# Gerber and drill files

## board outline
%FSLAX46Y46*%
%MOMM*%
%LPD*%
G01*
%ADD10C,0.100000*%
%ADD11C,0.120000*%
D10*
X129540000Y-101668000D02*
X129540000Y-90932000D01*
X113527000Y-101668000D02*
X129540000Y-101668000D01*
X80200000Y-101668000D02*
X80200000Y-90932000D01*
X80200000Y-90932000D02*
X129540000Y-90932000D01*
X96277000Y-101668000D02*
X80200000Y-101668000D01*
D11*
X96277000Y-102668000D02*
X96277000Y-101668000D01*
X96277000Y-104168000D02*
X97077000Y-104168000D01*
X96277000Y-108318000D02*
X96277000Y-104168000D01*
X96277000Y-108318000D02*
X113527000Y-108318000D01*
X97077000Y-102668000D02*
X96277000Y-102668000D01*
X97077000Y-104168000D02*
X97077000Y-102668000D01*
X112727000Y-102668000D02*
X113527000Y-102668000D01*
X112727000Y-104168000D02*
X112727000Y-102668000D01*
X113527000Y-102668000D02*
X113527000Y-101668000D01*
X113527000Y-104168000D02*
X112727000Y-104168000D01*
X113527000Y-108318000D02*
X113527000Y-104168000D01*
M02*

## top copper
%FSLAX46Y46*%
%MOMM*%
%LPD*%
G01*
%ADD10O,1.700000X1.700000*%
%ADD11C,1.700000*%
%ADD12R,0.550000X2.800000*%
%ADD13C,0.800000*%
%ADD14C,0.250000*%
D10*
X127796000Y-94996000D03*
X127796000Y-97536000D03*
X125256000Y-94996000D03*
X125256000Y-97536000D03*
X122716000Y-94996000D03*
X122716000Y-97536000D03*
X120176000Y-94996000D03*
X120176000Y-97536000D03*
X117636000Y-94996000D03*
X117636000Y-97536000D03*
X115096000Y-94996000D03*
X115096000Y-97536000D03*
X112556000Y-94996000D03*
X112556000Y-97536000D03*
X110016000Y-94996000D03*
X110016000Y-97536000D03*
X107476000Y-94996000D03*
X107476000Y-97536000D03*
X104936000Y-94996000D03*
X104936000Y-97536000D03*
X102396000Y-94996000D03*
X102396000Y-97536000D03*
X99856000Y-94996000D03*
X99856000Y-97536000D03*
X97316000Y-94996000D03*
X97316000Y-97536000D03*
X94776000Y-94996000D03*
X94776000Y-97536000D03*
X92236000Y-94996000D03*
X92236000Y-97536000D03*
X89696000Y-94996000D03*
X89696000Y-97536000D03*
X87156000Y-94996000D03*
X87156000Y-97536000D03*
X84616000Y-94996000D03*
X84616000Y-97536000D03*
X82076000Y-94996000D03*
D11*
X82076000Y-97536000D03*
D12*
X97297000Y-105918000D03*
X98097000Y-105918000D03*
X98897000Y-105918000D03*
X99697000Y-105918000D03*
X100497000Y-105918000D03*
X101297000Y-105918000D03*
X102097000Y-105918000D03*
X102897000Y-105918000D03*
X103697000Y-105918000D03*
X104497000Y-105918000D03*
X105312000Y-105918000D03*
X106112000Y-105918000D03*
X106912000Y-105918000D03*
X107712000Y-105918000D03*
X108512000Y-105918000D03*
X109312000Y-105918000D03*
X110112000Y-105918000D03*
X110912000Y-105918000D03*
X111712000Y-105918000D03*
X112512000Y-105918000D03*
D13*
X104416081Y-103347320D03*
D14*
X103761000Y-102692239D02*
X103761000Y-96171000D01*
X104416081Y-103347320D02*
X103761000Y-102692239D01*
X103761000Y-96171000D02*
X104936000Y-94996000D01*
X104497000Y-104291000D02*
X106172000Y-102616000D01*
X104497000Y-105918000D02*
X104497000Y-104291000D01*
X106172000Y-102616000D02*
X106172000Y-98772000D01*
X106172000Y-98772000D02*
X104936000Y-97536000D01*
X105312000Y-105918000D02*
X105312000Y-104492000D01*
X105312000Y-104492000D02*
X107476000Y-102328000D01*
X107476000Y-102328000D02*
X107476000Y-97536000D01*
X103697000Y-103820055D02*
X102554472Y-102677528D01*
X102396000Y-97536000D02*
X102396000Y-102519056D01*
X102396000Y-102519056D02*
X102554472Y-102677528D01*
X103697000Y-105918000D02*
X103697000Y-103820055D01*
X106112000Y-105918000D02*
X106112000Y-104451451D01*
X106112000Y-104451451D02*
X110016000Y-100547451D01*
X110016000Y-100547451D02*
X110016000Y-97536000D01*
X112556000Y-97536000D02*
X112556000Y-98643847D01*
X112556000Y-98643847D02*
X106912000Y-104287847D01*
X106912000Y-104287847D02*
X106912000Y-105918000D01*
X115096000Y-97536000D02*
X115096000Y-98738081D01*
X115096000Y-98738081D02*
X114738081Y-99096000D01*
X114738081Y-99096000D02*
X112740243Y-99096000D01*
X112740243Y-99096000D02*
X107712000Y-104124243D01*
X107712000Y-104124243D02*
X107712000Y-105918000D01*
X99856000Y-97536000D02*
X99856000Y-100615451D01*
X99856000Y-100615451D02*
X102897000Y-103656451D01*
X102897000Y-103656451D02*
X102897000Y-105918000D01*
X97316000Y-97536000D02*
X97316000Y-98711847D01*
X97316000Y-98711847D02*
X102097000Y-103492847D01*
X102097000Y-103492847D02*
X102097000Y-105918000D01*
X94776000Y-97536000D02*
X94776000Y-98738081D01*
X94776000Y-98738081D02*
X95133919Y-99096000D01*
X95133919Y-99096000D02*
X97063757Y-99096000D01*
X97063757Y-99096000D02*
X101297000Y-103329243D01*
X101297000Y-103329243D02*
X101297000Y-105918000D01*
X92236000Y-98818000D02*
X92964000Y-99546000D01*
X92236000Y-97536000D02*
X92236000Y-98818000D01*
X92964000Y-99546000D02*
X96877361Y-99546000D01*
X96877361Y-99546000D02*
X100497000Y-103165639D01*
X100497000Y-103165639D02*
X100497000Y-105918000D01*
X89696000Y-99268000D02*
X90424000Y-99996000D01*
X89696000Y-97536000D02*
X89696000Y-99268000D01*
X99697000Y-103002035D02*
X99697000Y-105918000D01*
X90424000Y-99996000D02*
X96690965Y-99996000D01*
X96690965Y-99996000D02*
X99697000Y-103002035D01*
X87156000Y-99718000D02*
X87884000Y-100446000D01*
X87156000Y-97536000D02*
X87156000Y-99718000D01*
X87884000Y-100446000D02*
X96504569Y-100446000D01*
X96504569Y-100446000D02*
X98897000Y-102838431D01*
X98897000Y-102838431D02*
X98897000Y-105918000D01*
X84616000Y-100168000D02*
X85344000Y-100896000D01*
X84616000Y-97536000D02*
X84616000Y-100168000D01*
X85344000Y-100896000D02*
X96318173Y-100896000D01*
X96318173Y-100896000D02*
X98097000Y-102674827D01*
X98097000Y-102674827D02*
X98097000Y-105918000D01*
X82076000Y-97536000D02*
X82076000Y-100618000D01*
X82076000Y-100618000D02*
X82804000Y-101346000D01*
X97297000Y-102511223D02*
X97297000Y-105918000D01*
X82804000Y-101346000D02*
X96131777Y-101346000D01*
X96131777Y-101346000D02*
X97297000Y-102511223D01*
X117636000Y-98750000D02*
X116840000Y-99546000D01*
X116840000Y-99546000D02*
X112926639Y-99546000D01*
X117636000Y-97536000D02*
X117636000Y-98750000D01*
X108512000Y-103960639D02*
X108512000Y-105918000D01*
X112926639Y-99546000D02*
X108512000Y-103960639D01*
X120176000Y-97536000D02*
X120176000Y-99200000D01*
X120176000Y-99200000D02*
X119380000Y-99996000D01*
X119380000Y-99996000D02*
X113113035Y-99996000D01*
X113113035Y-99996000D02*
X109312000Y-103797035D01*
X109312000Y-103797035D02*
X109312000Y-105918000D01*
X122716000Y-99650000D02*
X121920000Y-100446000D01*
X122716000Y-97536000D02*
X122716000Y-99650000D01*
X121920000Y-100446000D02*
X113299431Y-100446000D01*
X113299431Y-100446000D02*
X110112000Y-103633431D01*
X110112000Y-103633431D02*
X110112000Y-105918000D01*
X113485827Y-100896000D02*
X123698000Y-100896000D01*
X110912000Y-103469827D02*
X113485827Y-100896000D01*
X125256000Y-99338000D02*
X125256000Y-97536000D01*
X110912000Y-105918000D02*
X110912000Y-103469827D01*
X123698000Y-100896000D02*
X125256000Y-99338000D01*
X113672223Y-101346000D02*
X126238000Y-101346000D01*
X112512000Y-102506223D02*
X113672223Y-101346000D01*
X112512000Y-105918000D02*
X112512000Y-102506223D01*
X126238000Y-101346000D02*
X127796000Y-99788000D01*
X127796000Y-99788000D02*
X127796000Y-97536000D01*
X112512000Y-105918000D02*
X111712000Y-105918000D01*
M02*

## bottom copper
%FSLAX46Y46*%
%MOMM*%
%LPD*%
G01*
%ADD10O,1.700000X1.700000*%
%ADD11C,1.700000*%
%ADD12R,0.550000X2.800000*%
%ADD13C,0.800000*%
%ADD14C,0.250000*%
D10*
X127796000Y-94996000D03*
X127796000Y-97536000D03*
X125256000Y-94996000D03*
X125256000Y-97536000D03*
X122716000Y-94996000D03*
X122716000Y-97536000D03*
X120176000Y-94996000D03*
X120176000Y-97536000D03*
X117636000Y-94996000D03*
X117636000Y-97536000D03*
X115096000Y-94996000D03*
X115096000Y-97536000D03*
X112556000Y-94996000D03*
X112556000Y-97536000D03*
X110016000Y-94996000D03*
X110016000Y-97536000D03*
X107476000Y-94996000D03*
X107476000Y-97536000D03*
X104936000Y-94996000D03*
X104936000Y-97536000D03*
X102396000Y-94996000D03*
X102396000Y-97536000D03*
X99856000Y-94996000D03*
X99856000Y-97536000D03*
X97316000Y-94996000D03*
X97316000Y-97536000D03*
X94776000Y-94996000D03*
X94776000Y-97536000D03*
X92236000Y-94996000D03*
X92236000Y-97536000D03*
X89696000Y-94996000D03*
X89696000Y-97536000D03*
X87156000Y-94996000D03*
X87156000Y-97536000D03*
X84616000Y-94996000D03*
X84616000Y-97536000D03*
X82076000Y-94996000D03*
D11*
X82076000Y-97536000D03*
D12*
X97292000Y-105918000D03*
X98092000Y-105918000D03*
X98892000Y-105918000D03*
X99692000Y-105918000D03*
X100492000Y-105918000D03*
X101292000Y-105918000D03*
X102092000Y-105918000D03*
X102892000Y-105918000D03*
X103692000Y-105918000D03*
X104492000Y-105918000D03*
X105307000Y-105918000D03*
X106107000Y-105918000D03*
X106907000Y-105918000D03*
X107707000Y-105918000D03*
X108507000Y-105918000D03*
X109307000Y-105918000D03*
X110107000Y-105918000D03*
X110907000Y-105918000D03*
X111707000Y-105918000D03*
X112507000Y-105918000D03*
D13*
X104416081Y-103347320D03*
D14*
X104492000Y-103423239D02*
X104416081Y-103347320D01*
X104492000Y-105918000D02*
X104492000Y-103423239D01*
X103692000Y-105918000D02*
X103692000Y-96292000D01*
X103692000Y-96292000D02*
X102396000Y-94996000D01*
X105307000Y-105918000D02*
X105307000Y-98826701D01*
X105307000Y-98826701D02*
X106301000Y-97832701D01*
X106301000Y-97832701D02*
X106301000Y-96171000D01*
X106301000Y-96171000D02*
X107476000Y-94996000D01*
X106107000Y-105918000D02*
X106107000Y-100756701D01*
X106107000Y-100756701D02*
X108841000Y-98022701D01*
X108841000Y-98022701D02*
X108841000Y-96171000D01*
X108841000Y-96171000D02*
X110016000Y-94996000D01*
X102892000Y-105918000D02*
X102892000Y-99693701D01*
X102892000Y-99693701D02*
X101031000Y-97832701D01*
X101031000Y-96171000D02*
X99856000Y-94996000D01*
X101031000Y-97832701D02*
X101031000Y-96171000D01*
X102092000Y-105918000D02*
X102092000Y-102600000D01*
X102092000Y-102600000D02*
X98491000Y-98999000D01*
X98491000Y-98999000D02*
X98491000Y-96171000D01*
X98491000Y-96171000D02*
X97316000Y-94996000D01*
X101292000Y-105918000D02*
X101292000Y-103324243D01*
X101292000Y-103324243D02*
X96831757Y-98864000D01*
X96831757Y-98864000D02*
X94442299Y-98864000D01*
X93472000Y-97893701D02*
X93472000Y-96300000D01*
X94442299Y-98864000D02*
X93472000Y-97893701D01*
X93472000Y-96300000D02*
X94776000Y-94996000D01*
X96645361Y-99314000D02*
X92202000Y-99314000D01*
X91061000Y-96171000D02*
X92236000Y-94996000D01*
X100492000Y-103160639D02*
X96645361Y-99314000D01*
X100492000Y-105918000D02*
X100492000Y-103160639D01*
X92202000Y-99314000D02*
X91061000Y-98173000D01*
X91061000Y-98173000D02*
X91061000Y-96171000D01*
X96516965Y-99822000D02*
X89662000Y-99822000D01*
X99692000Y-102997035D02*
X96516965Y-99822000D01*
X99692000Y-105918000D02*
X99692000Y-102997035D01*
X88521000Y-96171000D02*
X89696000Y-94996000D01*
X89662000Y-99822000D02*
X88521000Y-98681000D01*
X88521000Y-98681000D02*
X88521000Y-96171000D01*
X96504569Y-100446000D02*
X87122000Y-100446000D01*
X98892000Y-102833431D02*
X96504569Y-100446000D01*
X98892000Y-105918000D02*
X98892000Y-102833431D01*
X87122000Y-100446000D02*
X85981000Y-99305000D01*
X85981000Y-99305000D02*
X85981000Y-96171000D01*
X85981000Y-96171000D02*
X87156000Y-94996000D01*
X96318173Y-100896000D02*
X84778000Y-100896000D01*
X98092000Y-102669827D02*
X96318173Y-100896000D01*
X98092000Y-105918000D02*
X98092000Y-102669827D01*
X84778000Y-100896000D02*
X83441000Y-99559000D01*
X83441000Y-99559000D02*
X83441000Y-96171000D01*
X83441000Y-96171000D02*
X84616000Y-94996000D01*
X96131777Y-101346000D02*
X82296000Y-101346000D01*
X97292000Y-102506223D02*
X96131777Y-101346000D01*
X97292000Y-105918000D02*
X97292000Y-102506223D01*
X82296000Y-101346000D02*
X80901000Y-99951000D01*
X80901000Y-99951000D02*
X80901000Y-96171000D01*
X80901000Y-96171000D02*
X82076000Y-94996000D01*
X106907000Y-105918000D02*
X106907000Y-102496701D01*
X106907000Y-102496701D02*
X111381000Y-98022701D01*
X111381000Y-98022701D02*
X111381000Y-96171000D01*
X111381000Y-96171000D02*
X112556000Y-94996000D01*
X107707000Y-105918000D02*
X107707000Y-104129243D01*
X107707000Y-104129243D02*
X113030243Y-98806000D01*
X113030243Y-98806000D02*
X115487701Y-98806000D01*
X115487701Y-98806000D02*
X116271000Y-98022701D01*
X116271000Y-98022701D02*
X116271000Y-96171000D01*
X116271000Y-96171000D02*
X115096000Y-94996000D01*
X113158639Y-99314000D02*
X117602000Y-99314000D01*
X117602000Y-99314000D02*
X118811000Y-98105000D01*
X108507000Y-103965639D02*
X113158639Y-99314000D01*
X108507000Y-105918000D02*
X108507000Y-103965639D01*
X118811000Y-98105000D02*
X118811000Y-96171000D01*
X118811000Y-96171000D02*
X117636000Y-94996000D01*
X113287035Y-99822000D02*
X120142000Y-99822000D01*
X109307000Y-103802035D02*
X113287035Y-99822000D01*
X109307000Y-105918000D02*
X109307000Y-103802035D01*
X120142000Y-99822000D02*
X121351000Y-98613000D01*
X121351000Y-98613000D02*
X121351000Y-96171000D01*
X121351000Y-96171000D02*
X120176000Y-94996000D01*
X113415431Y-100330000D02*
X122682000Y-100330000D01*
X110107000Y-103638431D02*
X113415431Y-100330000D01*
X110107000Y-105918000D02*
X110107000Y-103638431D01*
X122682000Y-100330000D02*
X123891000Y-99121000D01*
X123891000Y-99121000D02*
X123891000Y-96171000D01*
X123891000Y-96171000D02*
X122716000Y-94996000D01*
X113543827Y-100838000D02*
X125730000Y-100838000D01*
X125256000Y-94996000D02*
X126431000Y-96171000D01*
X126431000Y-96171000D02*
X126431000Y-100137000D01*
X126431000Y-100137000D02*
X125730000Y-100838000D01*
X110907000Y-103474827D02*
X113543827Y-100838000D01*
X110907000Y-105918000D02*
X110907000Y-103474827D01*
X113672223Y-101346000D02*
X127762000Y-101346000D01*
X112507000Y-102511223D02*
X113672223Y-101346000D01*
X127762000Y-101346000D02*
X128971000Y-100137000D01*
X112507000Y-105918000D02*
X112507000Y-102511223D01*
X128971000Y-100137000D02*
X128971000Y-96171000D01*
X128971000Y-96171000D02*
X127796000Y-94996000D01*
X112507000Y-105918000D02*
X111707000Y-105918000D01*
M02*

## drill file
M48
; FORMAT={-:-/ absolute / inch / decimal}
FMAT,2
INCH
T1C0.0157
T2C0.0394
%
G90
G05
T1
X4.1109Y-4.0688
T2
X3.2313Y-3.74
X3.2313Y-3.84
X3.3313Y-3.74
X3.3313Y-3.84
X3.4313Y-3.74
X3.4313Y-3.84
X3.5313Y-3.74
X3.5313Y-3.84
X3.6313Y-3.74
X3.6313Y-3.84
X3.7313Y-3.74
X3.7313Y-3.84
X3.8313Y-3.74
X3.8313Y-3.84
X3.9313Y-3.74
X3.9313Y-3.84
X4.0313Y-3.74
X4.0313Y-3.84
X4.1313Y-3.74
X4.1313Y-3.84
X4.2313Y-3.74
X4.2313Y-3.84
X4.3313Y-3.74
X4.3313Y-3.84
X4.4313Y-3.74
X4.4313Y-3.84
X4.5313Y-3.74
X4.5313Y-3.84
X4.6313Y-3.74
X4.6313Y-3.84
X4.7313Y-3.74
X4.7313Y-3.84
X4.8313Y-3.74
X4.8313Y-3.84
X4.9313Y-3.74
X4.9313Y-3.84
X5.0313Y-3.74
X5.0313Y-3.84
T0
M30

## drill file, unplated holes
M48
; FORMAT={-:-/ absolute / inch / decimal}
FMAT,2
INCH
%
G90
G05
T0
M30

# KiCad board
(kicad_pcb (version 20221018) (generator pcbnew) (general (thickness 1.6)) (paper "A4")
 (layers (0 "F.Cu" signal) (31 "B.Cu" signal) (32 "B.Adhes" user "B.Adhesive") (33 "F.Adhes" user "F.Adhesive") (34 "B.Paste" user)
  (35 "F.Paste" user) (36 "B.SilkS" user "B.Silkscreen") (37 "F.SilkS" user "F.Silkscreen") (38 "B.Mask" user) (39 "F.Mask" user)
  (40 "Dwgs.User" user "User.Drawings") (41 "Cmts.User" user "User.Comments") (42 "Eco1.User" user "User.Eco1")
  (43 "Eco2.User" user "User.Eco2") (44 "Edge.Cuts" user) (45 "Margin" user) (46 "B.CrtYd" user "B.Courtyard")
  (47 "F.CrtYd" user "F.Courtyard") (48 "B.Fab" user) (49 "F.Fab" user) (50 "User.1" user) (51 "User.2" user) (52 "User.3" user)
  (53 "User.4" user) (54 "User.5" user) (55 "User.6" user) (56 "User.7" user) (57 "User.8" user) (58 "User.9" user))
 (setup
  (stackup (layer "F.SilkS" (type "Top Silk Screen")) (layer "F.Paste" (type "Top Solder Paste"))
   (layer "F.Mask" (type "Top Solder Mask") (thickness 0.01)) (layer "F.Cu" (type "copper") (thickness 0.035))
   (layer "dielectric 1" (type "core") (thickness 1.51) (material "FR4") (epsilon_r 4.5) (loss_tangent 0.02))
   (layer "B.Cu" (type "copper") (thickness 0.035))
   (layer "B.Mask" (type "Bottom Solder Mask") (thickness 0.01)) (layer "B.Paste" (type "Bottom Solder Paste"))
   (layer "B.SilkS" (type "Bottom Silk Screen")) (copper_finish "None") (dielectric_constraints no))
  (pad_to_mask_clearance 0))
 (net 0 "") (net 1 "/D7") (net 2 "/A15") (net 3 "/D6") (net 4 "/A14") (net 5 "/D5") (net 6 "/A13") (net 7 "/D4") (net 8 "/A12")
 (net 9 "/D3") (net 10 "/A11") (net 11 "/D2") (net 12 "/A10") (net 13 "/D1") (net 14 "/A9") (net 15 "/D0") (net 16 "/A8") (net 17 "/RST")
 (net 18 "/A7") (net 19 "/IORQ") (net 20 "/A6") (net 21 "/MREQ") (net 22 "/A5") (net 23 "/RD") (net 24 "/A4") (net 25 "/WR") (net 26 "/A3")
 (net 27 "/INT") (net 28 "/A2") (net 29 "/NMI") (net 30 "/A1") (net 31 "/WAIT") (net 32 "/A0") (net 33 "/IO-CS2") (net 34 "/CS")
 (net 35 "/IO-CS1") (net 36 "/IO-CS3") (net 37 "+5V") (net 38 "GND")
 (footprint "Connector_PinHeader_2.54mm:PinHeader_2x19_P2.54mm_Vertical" (layer "F.Cu") (at 82.076 97.536 90)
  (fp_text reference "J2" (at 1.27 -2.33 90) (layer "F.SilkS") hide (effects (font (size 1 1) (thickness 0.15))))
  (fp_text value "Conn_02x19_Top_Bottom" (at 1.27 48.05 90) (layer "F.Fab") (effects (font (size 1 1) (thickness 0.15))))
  (pad "1" thru_hole circle (at 0 0 90) (size 1.7 1.7) (drill 1) (layers "*.Cu" "*.Mask") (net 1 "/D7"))
  (pad "2" thru_hole oval (at 2.54 0 90) (size 1.7 1.7) (drill 1) (layers "*.Cu" "*.Mask") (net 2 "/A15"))
  (pad "3" thru_hole oval (at 0 2.54 90) (size 1.7 1.7) (drill 1) (layers "*.Cu" "*.Mask") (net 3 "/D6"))
  (pad "4" thru_hole oval (at 2.54 2.54 90) (size 1.7 1.7) (drill 1) (layers "*.Cu" "*.Mask") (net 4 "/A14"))
  (pad "5" thru_hole oval (at 0 5.08 90) (size 1.7 1.7) (drill 1) (layers "*.Cu" "*.Mask") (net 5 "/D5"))
  (pad "6" thru_hole oval (at 2.54 5.08 90) (size 1.7 1.7) (drill 1) (layers "*.Cu" "*.Mask") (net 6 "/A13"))
  (pad "7" thru_hole oval (at 0 7.62 90) (size 1.7 1.7) (drill 1) (layers "*.Cu" "*.Mask") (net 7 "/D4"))
  (pad "8" thru_hole oval (at 2.54 7.62 90) (size 1.7 1.7) (drill 1) (layers "*.Cu" "*.Mask") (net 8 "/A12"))
  (pad "9" thru_hole oval (at 0 10.16 90) (size 1.7 1.7) (drill 1) (layers "*.Cu" "*.Mask") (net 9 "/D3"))
  (pad "10" thru_hole oval (at 2.54 10.16 90) (size 1.7 1.7) (drill 1) (layers "*.Cu" "*.Mask") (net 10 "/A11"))
  (pad "11" thru_hole oval (at 0 12.7 90) (size 1.7 1.7) (drill 1) (layers "*.Cu" "*.Mask") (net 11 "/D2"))
  (pad "12" thru_hole oval (at 2.54 12.7 90) (size 1.7 1.7) (drill 1) (layers "*.Cu" "*.Mask") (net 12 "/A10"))
  (pad "13" thru_hole oval (at 0 15.24 90) (size 1.7 1.7) (drill 1) (layers "*.Cu" "*.Mask") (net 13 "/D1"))
  (pad "14" thru_hole oval (at 2.54 15.24 90) (size 1.7 1.7) (drill 1) (layers "*.Cu" "*.Mask") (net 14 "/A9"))
  (pad "15" thru_hole oval (at 0 17.78 90) (size 1.7 1.7) (drill 1) (layers "*.Cu" "*.Mask") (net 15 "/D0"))
  (pad "16" thru_hole oval (at 2.54 17.78 90) (size 1.7 1.7) (drill 1) (layers "*.Cu" "*.Mask") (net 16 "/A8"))
  (pad "17" thru_hole oval (at 0 20.32 90) (size 1.7 1.7) (drill 1) (layers "*.Cu" "*.Mask") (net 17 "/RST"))
  (pad "18" thru_hole oval (at 2.54 20.32 90) (size 1.7 1.7) (drill 1) (layers "*.Cu" "*.Mask") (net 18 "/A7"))
  (pad "19" thru_hole oval (at 0 22.86 90) (size 1.7 1.7) (drill 1) (layers "*.Cu" "*.Mask") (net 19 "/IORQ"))
  (pad "20" thru_hole oval (at 2.54 22.86 90) (size 1.7 1.7) (drill 1) (layers "*.Cu" "*.Mask") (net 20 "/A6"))
  (pad "21" thru_hole oval (at 0 25.4 90) (size 1.7 1.7) (drill 1) (layers "*.Cu" "*.Mask") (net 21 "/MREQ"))
  (pad "22" thru_hole oval (at 2.54 25.4 90) (size 1.7 1.7) (drill 1) (layers "*.Cu" "*.Mask") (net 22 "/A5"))
  (pad "23" thru_hole oval (at 0 27.94 90) (size 1.7 1.7) (drill 1) (layers "*.Cu" "*.Mask") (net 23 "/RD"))
  (pad "24" thru_hole oval (at 2.54 27.94 90) (size 1.7 1.7) (drill 1) (layers "*.Cu" "*.Mask") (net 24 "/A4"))
  (pad "25" thru_hole oval (at 0 30.48 90) (size 1.7 1.7) (drill 1) (layers "*.Cu" "*.Mask") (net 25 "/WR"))
  (pad "26" thru_hole oval (at 2.54 30.48 90) (size 1.7 1.7) (drill 1) (layers "*.Cu" "*.Mask") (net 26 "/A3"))
  (pad "27" thru_hole oval (at 0 33.02 90) (size 1.7 1.7) (drill 1) (layers "*.Cu" "*.Mask") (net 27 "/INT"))
  (pad "28" thru_hole oval (at 2.54 33.02 90) (size 1.7 1.7) (drill 1) (layers "*.Cu" "*.Mask") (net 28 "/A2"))
  (pad "29" thru_hole oval (at 0 35.56 90) (size 1.7 1.7) (drill 1) (layers "*.Cu" "*.Mask") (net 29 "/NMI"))
  (pad "30" thru_hole oval (at 2.54 35.56 90) (size 1.7 1.7) (drill 1) (layers "*.Cu" "*.Mask") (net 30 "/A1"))
  (pad "31" thru_hole oval (at 0 38.1 90) (size 1.7 1.7) (drill 1) (layers "*.Cu" "*.Mask") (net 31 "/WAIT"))
  (pad "32" thru_hole oval (at 2.54 38.1 90) (size 1.7 1.7) (drill 1) (layers "*.Cu" "*.Mask") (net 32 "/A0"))
  (pad "33" thru_hole oval (at 0 40.64 90) (size 1.7 1.7) (drill 1) (layers "*.Cu" "*.Mask") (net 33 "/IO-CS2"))
  (pad "34" thru_hole oval (at 2.54 40.64 90) (size 1.7 1.7) (drill 1) (layers "*.Cu" "*.Mask") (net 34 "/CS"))
  (pad "35" thru_hole oval (at 0 43.18 90) (size 1.7 1.7) (drill 1) (layers "*.Cu" "*.Mask") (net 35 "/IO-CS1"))
  (pad "36" thru_hole oval (at 2.54 43.18 90) (size 1.7 1.7) (drill 1) (layers "*.Cu" "*.Mask") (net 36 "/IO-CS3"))
  (pad "37" thru_hole oval (at 0 45.72 90) (size 1.7 1.7) (drill 1) (layers "*.Cu" "*.Mask") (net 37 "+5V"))
  (pad "38" thru_hole oval (at 2.54 45.72 90) (size 1.7 1.7) (drill 1) (layers "*.Cu" "*.Mask") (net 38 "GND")))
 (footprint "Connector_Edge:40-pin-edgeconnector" (layer "F.Cu") (at 104.902 103.378)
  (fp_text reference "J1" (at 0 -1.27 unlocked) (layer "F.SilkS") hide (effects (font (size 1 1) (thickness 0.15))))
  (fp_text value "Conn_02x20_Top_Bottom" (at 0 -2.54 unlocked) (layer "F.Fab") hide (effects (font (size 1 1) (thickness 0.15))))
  (fp_line (start -8.625 -0.71) (end -8.625 -1.71) (stroke (width 0.12) (type default)) (layer "Edge.Cuts"))
  (fp_line (start -8.625 0.79) (end -7.825 0.79) (stroke (width 0.12) (type default)) (layer "Edge.Cuts"))
  (fp_line (start -8.625 4.94) (end -8.625 0.79) (stroke (width 0.12) (type default)) (layer "Edge.Cuts"))
  (fp_line (start -8.625 4.94) (end 8.625 4.94) (stroke (width 0.12) (type default)) (layer "Edge.Cuts"))
  (fp_line (start -7.825 -0.71) (end -8.625 -0.71) (stroke (width 0.12) (type default)) (layer "Edge.Cuts"))
  (fp_line (start -7.825 0.79) (end -7.825 -0.71) (stroke (width 0.12) (type default)) (layer "Edge.Cuts"))
  (fp_line (start 7.825 -0.71) (end 8.625 -0.71) (stroke (width 0.12) (type default)) (layer "Edge.Cuts"))
  (fp_line (start 7.825 0.79) (end 7.825 -0.71) (stroke (width 0.12) (type default)) (layer "Edge.Cuts"))
  (fp_line (start 8.625 -0.71) (end 8.625 -1.71) (stroke (width 0.12) (type default)) (layer "Edge.Cuts"))
  (fp_line (start 8.625 0.79) (end 7.825 0.79) (stroke (width 0.12) (type default)) (layer "Edge.Cuts"))
  (fp_line (start 8.625 4.94) (end 8.625 0.79) (stroke (width 0.12) (type default)) (layer "Edge.Cuts"))
  (pad "1" smd rect (at -7.605 2.54 90) (size 2.8 0.55) (layers "F.Cu" "F.Paste" "F.Mask") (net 1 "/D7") (thermal_bridge_angle 45))
  (pad "2" smd rect (at -6.805 2.54 90) (size 2.8 0.55) (layers "F.Cu" "F.Paste" "F.Mask") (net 3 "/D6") (thermal_bridge_angle 45))
  (pad "3" smd rect (at -6.005 2.54 90) (size 2.8 0.55) (layers "F.Cu" "F.Paste" "F.Mask") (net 5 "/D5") (thermal_bridge_angle 45))
  (pad "4" smd rect (at -5.205 2.54 90) (size 2.8 0.55) (layers "F.Cu" "F.Paste" "F.Mask") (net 7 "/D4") (thermal_bridge_angle 45))
  (pad "5" smd rect (at -4.405 2.54 90) (size 2.8 0.55) (layers "F.Cu" "F.Paste" "F.Mask") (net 9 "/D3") (thermal_bridge_angle 45))
  (pad "6" smd rect (at -3.605 2.54 90) (size 2.8 0.55) (layers "F.Cu" "F.Paste" "F.Mask") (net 11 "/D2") (thermal_bridge_angle 45))
  (pad "7" smd rect (at -2.805 2.54 90) (size 2.8 0.55) (layers "F.Cu" "F.Paste" "F.Mask") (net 13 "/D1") (thermal_bridge_angle 45))
  (pad "8" smd rect (at -2.005 2.54 90) (size 2.8 0.55) (layers "F.Cu" "F.Paste" "F.Mask") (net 15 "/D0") (thermal_bridge_angle 45))
  (pad "9" smd rect (at -1.205 2.54 90) (size 2.8 0.55) (layers "F.Cu" "F.Paste" "F.Mask") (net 17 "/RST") (thermal_bridge_angle 45))
  (pad "10" smd rect (at -0.405 2.54 90) (size 2.8 0.55) (layers "F.Cu" "F.Paste" "F.Mask") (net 19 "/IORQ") (thermal_bridge_angle 45))
  (pad "11" smd rect (at 0.41 2.54 90) (size 2.8 0.55) (layers "F.Cu" "F.Paste" "F.Mask") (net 21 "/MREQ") (thermal_bridge_angle 45))
  (pad "12" smd rect (at 1.21 2.54 90) (size 2.8 0.55) (layers "F.Cu" "F.Paste" "F.Mask") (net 23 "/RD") (thermal_bridge_angle 45))
  (pad "13" smd rect (at 2.01 2.54 90) (size 2.8 0.55) (layers "F.Cu" "F.Paste" "F.Mask") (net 25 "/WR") (thermal_bridge_angle 45))
  (pad "14" smd rect (at 2.81 2.54 90) (size 2.8 0.55) (layers "F.Cu" "F.Paste" "F.Mask") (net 27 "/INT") (thermal_bridge_angle 45))
  (pad "15" smd rect (at 3.61 2.54 90) (size 2.8 0.55) (layers "F.Cu" "F.Paste" "F.Mask") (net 29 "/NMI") (thermal_bridge_angle 45))
  (pad "16" smd rect (at 4.41 2.54 90) (size 2.8 0.55) (layers "F.Cu" "F.Paste" "F.Mask") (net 31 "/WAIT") (thermal_bridge_angle 45))
  (pad "17" smd rect (at 5.21 2.54 90) (size 2.8 0.55) (layers "F.Cu" "F.Paste" "F.Mask") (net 33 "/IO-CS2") (thermal_bridge_angle 45))
  (pad "18" smd rect (at 6.01 2.54 90) (size 2.8 0.55) (layers "F.Cu" "F.Paste" "F.Mask") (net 35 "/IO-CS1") (thermal_bridge_angle 45))
  (pad "19" smd rect (at 6.81 2.54 90) (size 2.8 0.55) (layers "F.Cu" "F.Paste" "F.Mask") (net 37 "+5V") (thermal_bridge_angle 45))
  (pad "20" smd rect (at 7.61 2.54 90) (size 2.8 0.55) (layers "F.Cu" "F.Paste" "F.Mask") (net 37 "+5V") (thermal_bridge_angle 45))
  (pad "21" smd rect (at -7.61 2.54 270) (size 2.8 0.55) (layers "B.Cu" "B.Paste" "B.Mask") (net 2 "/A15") (thermal_bridge_angle 45))
  (pad "22" smd rect (at -6.81 2.54 270) (size 2.8 0.55) (layers "B.Cu" "B.Paste" "B.Mask") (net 4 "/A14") (thermal_bridge_angle 45))
  (pad "23" smd rect (at -6.01 2.54 270) (size 2.8 0.55) (layers "B.Cu" "B.Paste" "B.Mask") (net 6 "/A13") (thermal_bridge_angle 45))
  (pad "24" smd rect (at -5.21 2.54 270) (size 2.8 0.55) (layers "B.Cu" "B.Paste" "B.Mask") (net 8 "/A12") (thermal_bridge_angle 45))
  (pad "25" smd rect (at -4.41 2.54 270) (size 2.8 0.55) (layers "B.Cu" "B.Paste" "B.Mask") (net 10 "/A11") (thermal_bridge_angle 45))
  (pad "26" smd rect (at -3.61 2.54 270) (size 2.8 0.55) (layers "B.Cu" "B.Paste" "B.Mask") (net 12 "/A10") (thermal_bridge_angle 45))
  (pad "27" smd rect (at -2.81 2.54 270) (size 2.8 0.55) (layers "B.Cu" "B.Paste" "B.Mask") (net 14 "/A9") (thermal_bridge_angle 45))
  (pad "28" smd rect (at -2.01 2.54 270) (size 2.8 0.55) (layers "B.Cu" "B.Paste" "B.Mask") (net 16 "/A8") (thermal_bridge_angle 45))
  (pad "29" smd rect (at -1.21 2.54 270) (size 2.8 0.55) (layers "B.Cu" "B.Paste" "B.Mask") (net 18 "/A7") (thermal_bridge_angle 45))
  (pad "30" smd rect (at -0.41 2.54 270) (size 2.8 0.55) (layers "B.Cu" "B.Paste" "B.Mask") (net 20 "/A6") (thermal_bridge_angle 45))
  (pad "31" smd rect (at 0.405 2.54 270) (size 2.8 0.55) (layers "B.Cu" "B.Paste" "B.Mask") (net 22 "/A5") (thermal_bridge_angle 45))
  (pad "32" smd rect (at 1.205 2.54 270) (size 2.8 0.55) (layers "B.Cu" "B.Paste" "B.Mask") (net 24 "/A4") (thermal_bridge_angle 45))
  (pad "33" smd rect (at 2.005 2.54 270) (size 2.8 0.55) (layers "B.Cu" "B.Paste" "B.Mask") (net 26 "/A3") (thermal_bridge_angle 45))
  (pad "34" smd rect (at 2.805 2.54 270) (size 2.8 0.55) (layers "B.Cu" "B.Paste" "B.Mask") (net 28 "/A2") (thermal_bridge_angle 45))
  (pad "35" smd rect (at 3.605 2.54 270) (size 2.8 0.55) (layers "B.Cu" "B.Paste" "B.Mask") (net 30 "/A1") (thermal_bridge_angle 45))
  (pad "36" smd rect (at 4.405 2.54 270) (size 2.8 0.55) (layers "B.Cu" "B.Paste" "B.Mask") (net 32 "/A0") (thermal_bridge_angle 45))
  (pad "37" smd rect (at 5.205 2.54 270) (size 2.8 0.55) (layers "B.Cu" "B.Paste" "B.Mask") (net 34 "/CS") (thermal_bridge_angle 45))
  (pad "38" smd rect (at 6.005 2.54 270) (size 2.8 0.55) (layers "B.Cu" "B.Paste" "B.Mask") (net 36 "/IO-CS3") (thermal_bridge_angle 45))
  (pad "39" smd rect (at 6.805 2.54 270) (size 2.8 0.55) (layers "B.Cu" "B.Paste" "B.Mask") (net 38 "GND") (thermal_bridge_angle 45))
  (pad "40" smd rect (at 7.605 2.54 270) (size 2.8 0.55) (layers "B.Cu" "B.Paste" "B.Mask") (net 38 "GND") (thermal_bridge_angle 45)))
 (gr_line (start 129.54 101.668) (end 129.54 90.932) (stroke (width 0.1) (type default)) (layer "Edge.Cuts"))
 (gr_line (start 113.527 101.668) (end 129.54 101.668) (stroke (width 0.1) (type default)) (layer "Edge.Cuts"))
 (gr_line (start 80.2 101.668) (end 80.2 90.932) (stroke (width 0.1) (type default)) (layer "Edge.Cuts"))
 (gr_line (start 80.2 90.932) (end 129.54 90.932) (stroke (width 0.1) (type default)) (layer "Edge.Cuts"))
 (gr_line (start 96.277 101.668) (end 80.2 101.668) (stroke (width 0.1) (type default)) (layer "Edge.Cuts"))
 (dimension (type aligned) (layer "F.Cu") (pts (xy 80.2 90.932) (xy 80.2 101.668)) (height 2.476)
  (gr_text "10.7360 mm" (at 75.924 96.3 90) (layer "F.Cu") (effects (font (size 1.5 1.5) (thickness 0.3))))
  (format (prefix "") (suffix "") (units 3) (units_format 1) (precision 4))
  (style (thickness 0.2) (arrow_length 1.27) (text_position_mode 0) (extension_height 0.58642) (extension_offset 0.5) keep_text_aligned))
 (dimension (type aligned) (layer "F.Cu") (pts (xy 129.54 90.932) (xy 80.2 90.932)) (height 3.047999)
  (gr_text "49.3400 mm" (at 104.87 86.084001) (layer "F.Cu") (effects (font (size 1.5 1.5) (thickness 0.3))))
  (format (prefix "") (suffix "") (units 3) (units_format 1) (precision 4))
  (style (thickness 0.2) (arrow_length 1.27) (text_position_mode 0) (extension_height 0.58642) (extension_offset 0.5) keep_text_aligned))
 (segment (start 82.076 97.536) (end 82.076 100.618) (width 0.25) (layer "F.Cu") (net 1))
 (segment (start 97.297 102.511223) (end 97.297 105.918) (width 0.25) (layer "F.Cu") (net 1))
 (segment (start 82.804 101.346) (end 96.131777 101.346) (width 0.25) (layer "F.Cu") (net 1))
 (segment (start 82.076 100.618) (end 82.804 101.346) (width 0.25) (layer "F.Cu") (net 1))
 (segment (start 96.131777 101.346) (end 97.297 102.511223) (width 0.25) (layer "F.Cu") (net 1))
 (segment (start 84.616 97.536) (end 84.616 100.168) (width 0.25) (layer "F.Cu") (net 3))
 (segment (start 96.318173 100.896) (end 98.097 102.674827) (width 0.25) (layer "F.Cu") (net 3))
 (segment (start 84.616 100.168) (end 85.344 100.896) (width 0.25) (layer "F.Cu") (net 3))
 (segment (start 85.344 100.896) (end 96.318173 100.896) (width 0.25) (layer "F.Cu") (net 3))
 (segment (start 98.097 102.674827) (end 98.097 105.918) (width 0.25) (layer "F.Cu") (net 3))
 (segment (start 87.156 99.718) (end 87.884 100.446) (width 0.25) (layer "F.Cu") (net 5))
 (segment (start 98.897 102.838431) (end 98.897 105.918) (width 0.25) (layer "F.Cu") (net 5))
 (segment (start 96.504569 100.446) (end 98.897 102.838431) (width 0.25) (layer "F.Cu") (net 5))
 (segment (start 87.156 97.536) (end 87.156 99.718) (width 0.25) (layer "F.Cu") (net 5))
 (segment (start 87.884 100.446) (end 96.504569 100.446) (width 0.25) (layer "F.Cu") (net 5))
 (segment (start 90.424 99.996) (end 96.690965 99.996) (width 0.25) (layer "F.Cu") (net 7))
 (segment (start 89.696 97.536) (end 89.696 99.268) (width 0.25) (layer "F.Cu") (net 7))
 (segment (start 89.696 99.268) (end 90.424 99.996) (width 0.25) (layer "F.Cu") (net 7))
 (segment (start 96.690965 99.996) (end 99.697 103.002035) (width 0.25) (layer "F.Cu") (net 7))
 (segment (start 99.697 103.002035) (end 99.697 105.918) (width 0.25) (layer "F.Cu") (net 7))
 (segment (start 92.964 99.546) (end 96.877361 99.546) (width 0.25) (layer "F.Cu") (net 9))
 (segment (start 92.236 98.818) (end 92.964 99.546) (width 0.25) (layer "F.Cu") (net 9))
 (segment (start 92.236 97.536) (end 92.236 98.818) (width 0.25) (layer "F.Cu") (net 9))
 (segment (start 100.497 103.165639) (end 100.497 105.918) (width 0.25) (layer "F.Cu") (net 9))
 (segment (start 96.877361 99.546) (end 100.497 103.165639) (width 0.25) (layer "F.Cu") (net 9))
 (segment (start 97.063757 99.096) (end 101.297 103.329243) (width 0.25) (layer "F.Cu") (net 11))
 (segment (start 95.133919 99.096) (end 97.063757 99.096) (width 0.25) (layer "F.Cu") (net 11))
 (segment (start 94.776 98.738081) (end 95.133919 99.096) (width 0.25) (layer "F.Cu") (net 11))
 (segment (start 94.776 97.536) (end 94.776 98.738081) (width 0.25) (layer "F.Cu") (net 11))
 (segment (start 101.297 103.329243) (end 101.297 105.918) (width 0.25) (layer "F.Cu") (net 11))
 (segment (start 97.316 98.711847) (end 102.097 103.492847) (width 0.25) (layer "F.Cu") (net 13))
 (segment (start 97.316 97.536) (end 97.316 98.711847) (width 0.25) (layer "F.Cu") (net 13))
 (segment (start 102.097 103.492847) (end 102.097 105.918) (width 0.25) (layer "F.Cu") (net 13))
 (segment (start 102.897 103.656451) (end 102.897 105.918) (width 0.25) (layer "F.Cu") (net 15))
 (segment (start 99.856 97.536) (end 99.856 100.615451) (width 0.25) (layer "F.Cu") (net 15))
 (segment (start 99.856 100.615451) (end 102.897 103.656451) (width 0.25) (layer "F.Cu") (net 15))
 (segment (start 103.697 103.820055) (end 102.554472 102.677528) (width 0.25) (layer "F.Cu") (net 17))
 (segment (start 102.396 97.536) (end 102.396 102.519056) (width 0.25) (layer "F.Cu") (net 17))
 (segment (start 102.396 102.519056) (end 102.554472 102.677528) (width 0.25) (layer "F.Cu") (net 17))
 (segment (start 103.697 105.918) (end 103.697 103.820055) (width 0.25) (layer "F.Cu") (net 17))
 (segment (start 104.497 104.291) (end 106.172 102.616) (width 0.25) (layer "F.Cu") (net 19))
 (segment (start 106.172 98.772) (end 104.936 97.536) (width 0.25) (layer "F.Cu") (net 19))
 (segment (start 104.497 105.918) (end 104.497 104.291) (width 0.25) (layer "F.Cu") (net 19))
 (segment (start 106.172 102.616) (end 106.172 98.772) (width 0.25) (layer "F.Cu") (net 19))
 (segment (start 107.476 102.328) (end 107.476 97.536) (width 0.25) (layer "F.Cu") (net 21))
 (segment (start 105.312 104.492) (end 107.476 102.328) (width 0.25) (layer "F.Cu") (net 21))
 (segment (start 105.312 105.918) (end 105.312 104.492) (width 0.25) (layer "F.Cu") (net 21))
 (segment (start 106.112 104.451451) (end 110.016 100.547451) (width 0.25) (layer "F.Cu") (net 23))
 (segment (start 106.112 105.918) (end 106.112 104.451451) (width 0.25) (layer "F.Cu") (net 23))
 (segment (start 110.016 100.547451) (end 110.016 97.536) (width 0.25) (layer "F.Cu") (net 23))
 (segment (start 112.556 97.536) (end 112.556 98.643847) (width 0.25) (layer "F.Cu") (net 25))
 (segment (start 106.912 104.287847) (end 106.912 105.918) (width 0.25) (layer "F.Cu") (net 25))
 (segment (start 112.556 98.643847) (end 106.912 104.287847) (width 0.25) (layer "F.Cu") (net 25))
 (segment (start 112.740243 99.096) (end 107.712 104.124243) (width 0.25) (layer "F.Cu") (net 27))
 (segment (start 115.096 97.536) (end 115.096 98.738081) (width 0.25) (layer "F.Cu") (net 27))
 (segment (start 114.738081 99.096) (end 112.740243 99.096) (width 0.25) (layer "F.Cu") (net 27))
 (segment (start 115.096 98.738081) (end 114.738081 99.096) (width 0.25) (layer "F.Cu") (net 27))
 (segment (start 107.712 104.124243) (end 107.712 105.918) (width 0.25) (layer "F.Cu") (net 27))
 (segment (start 112.926639 99.546) (end 108.512 103.960639) (width 0.25) (layer "F.Cu") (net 29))
 (segment (start 117.636 98.75) (end 116.84 99.546) (width 0.25) (layer "F.Cu") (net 29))
 (segment (start 116.84 99.546) (end 112.926639 99.546) (width 0.25) (layer "F.Cu") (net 29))
 (segment (start 117.636 97.536) (end 117.636 98.75) (width 0.25) (layer "F.Cu") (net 29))
 (segment (start 108.512 103.960639) (end 108.512 105.918) (width 0.25) (layer "F.Cu") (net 29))
 (segment (start 120.176 99.2) (end 119.38 99.996) (width 0.25) (layer "F.Cu") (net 31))
 (segment (start 109.312 103.797035) (end 109.312 105.918) (width 0.25) (layer "F.Cu") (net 31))
 (segment (start 120.176 97.536) (end 120.176 99.2) (width 0.25) (layer "F.Cu") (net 31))
 (segment (start 119.38 99.996) (end 113.113035 99.996) (width 0.25) (layer "F.Cu") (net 31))
 (segment (start 113.113035 99.996) (end 109.312 103.797035) (width 0.25) (layer "F.Cu") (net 31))
 (segment (start 110.112 103.633431) (end 110.112 105.918) (width 0.25) (layer "F.Cu") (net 33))
 (segment (start 113.299431 100.446) (end 110.112 103.633431) (width 0.25) (layer "F.Cu") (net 33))
 (segment (start 121.92 100.446) (end 113.299431 100.446) (width 0.25) (layer "F.Cu") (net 33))
 (segment (start 122.716 99.65) (end 121.92 100.446) (width 0.25) (layer "F.Cu") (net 33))
 (segment (start 122.716 97.536) (end 122.716 99.65) (width 0.25) (layer "F.Cu") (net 33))
 (segment (start 125.256 99.338) (end 125.256 97.536) (width 0.25) (layer "F.Cu") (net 35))
 (segment (start 113.485827 100.896) (end 123.698 100.896) (width 0.25) (layer "F.Cu") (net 35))
 (segment (start 123.698 100.896) (end 125.256 99.338) (width 0.25) (layer "F.Cu") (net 35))
 (segment (start 110.912 105.918) (end 110.912 103.469827) (width 0.25) (layer "F.Cu") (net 35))
 (segment (start 110.912 103.469827) (end 113.485827 100.896) (width 0.25) (layer "F.Cu") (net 35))
 (segment (start 112.512 105.918) (end 111.712 105.918) (width 0.25) (layer "F.Cu") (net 37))
 (segment (start 126.238 101.346) (end 127.796 99.788) (width 0.25) (layer "F.Cu") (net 37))
 (segment (start 127.796 99.788) (end 127.796 97.536) (width 0.25) (layer "F.Cu") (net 37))
 (segment (start 112.512 105.918) (end 112.512 102.506223) (width 0.25) (layer "F.Cu") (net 37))
 (segment (start 113.672223 101.346) (end 126.238 101.346) (width 0.25) (layer "F.Cu") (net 37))
 (segment (start 112.512 102.506223) (end 113.672223 101.346) (width 0.25) (layer "F.Cu") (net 37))
 (segment (start 97.292 102.506223) (end 96.131777 101.346) (width 0.25) (layer "B.Cu") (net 2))
 (segment (start 97.292 105.918) (end 97.292 102.506223) (width 0.25) (layer "B.Cu") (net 2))
 (segment (start 80.901 99.951) (end 80.901 96.171) (width 0.25) (layer "B.Cu") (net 2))
 (segment (start 96.131777 101.346) (end 82.296 101.346) (width 0.25) (layer "B.Cu") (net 2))
 (segment (start 82.296 101.346) (end 80.901 99.951) (width 0.25) (layer "B.Cu") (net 2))
 (segment (start 80.901 96.171) (end 82.076 94.996) (width 0.25) (layer "B.Cu") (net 2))
 (segment (start 84.778 100.896) (end 83.441 99.559) (width 0.25) (layer "B.Cu") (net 4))
 (segment (start 96.318173 100.896) (end 84.778 100.896) (width 0.25) (layer "B.Cu") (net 4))
 (segment (start 83.441 96.171) (end 84.616 94.996) (width 0.25) (layer "B.Cu") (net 4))
 (segment (start 98.092 102.669827) (end 96.318173 100.896) (width 0.25) (layer "B.Cu") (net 4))
 (segment (start 83.441 99.559) (end 83.441 96.171) (width 0.25) (layer "B.Cu") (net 4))
 (segment (start 98.092 105.918) (end 98.092 102.669827) (width 0.25) (layer "B.Cu") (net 4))
 (segment (start 96.504569 100.446) (end 87.122 100.446) (width 0.25) (layer "B.Cu") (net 6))
 (segment (start 85.981 99.305) (end 85.981 96.171) (width 0.25) (layer "B.Cu") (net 6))
 (segment (start 98.892 102.833431) (end 96.504569 100.446) (width 0.25) (layer "B.Cu") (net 6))
 (segment (start 87.122 100.446) (end 85.981 99.305) (width 0.25) (layer "B.Cu") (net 6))
 (segment (start 85.981 96.171) (end 87.156 94.996) (width 0.25) (layer "B.Cu") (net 6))
 (segment (start 98.892 105.918) (end 98.892 102.833431) (width 0.25) (layer "B.Cu") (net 6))
 (segment (start 99.692 102.997035) (end 96.516965 99.822) (width 0.25) (layer "B.Cu") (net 8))
 (segment (start 96.516965 99.822) (end 89.662 99.822) (width 0.25) (layer "B.Cu") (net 8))
 (segment (start 99.692 105.918) (end 99.692 102.997035) (width 0.25) (layer "B.Cu") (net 8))
 (segment (start 88.521 98.681) (end 88.521 96.171) (width 0.25) (layer "B.Cu") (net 8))
 (segment (start 88.521 96.171) (end 89.696 94.996) (width 0.25) (layer "B.Cu") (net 8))
 (segment (start 89.662 99.822) (end 88.521 98.681) (width 0.25) (layer "B.Cu") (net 8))
 (segment (start 100.492 103.160639) (end 96.645361 99.314) (width 0.25) (layer "B.Cu") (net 10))
 (segment (start 91.061 98.173) (end 91.061 96.171) (width 0.25) (layer "B.Cu") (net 10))
 (segment (start 96.645361 99.314) (end 92.202 99.314) (width 0.25) (layer "B.Cu") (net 10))
 (segment (start 92.202 99.314) (end 91.061 98.173) (width 0.25) (layer "B.Cu") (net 10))
 (segment (start 100.492 105.918) (end 100.492 103.160639) (width 0.25) (layer "B.Cu") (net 10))
 (segment (start 91.061 96.171) (end 92.236 94.996) (width 0.25) (layer "B.Cu") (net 10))
 (segment (start 101.292 105.918) (end 101.292 103.324243) (width 0.25) (layer "B.Cu") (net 12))
 (segment (start 94.442299 98.864) (end 93.472 97.893701) (width 0.25) (layer "B.Cu") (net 12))
 (segment (start 101.292 103.324243) (end 96.831757 98.864) (width 0.25) (layer "B.Cu") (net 12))
 (segment (start 93.472 96.3) (end 94.776 94.996) (width 0.25) (layer "B.Cu") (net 12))
 (segment (start 96.831757 98.864) (end 94.442299 98.864) (width 0.25) (layer "B.Cu") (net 12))
 (segment (start 93.472 97.893701) (end 93.472 96.3) (width 0.25) (layer "B.Cu") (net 12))
 (segment (start 102.092 105.918) (end 102.092 102.6) (width 0.25) (layer "B.Cu") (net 14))
 (segment (start 98.491 98.999) (end 98.491 96.171) (width 0.25) (layer "B.Cu") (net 14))
 (segment (start 102.092 102.6) (end 98.491 98.999) (width 0.25) (layer "B.Cu") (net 14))
 (segment (start 98.491 96.171) (end 97.316 94.996) (width 0.25) (layer "B.Cu") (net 14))
 (segment (start 101.031 97.832701) (end 101.031 96.171) (width 0.25) (layer "B.Cu") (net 16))
 (segment (start 101.031 96.171) (end 99.856 94.996) (width 0.25) (layer "B.Cu") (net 16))
 (segment (start 102.892 105.918) (end 102.892 99.693701) (width 0.25) (layer "B.Cu") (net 16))
 (segment (start 102.892 99.693701) (end 101.031 97.832701) (width 0.25) (layer "B.Cu") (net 16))
 (segment (start 103.692 96.292) (end 102.396 94.996) (width 0.25) (layer "B.Cu") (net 18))
 (segment (start 103.692 105.918) (end 103.692 96.292) (width 0.25) (layer "B.Cu") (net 18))
 (segment (start 103.761 102.692239) (end 103.761 96.171) (width 0.25) (layer "F.Cu") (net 20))
 (segment (start 104.416081 103.34732) (end 103.761 102.692239) (width 0.25) (layer "F.Cu") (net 20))
 (segment (start 103.761 96.171) (end 104.936 94.996) (width 0.25) (layer "F.Cu") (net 20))
 (via (at 104.416081 103.34732) (size 0.8) (drill 0.4) (layers "F.Cu" "B.Cu") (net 20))
 (segment (start 104.492 103.423239) (end 104.416081 103.34732) (width 0.25) (layer "B.Cu") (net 20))
 (segment (start 104.492 105.918) (end 104.492 103.423239) (width 0.25) (layer "B.Cu") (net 20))
 (segment (start 105.307 98.826701) (end 106.301 97.832701) (width 0.25) (layer "B.Cu") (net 22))
 (segment (start 106.301 96.171) (end 107.476 94.996) (width 0.25) (layer "B.Cu") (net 22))
 (segment (start 105.307 105.918) (end 105.307 98.826701) (width 0.25) (layer "B.Cu") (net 22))
 (segment (start 106.301 97.832701) (end 106.301 96.171) (width 0.25) (layer "B.Cu") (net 22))
 (segment (start 108.841 98.022701) (end 108.841 96.171) (width 0.25) (layer "B.Cu") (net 24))
 (segment (start 108.841 96.171) (end 110.016 94.996) (width 0.25) (layer "B.Cu") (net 24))
 (segment (start 106.107 105.918) (end 106.107 100.756701) (width 0.25) (layer "B.Cu") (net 24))
 (segment (start 106.107 100.756701) (end 108.841 98.022701) (width 0.25) (layer "B.Cu") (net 24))
 (segment (start 106.907 102.496701) (end 111.381 98.022701) (width 0.25) (layer "B.Cu") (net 26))
 (segment (start 106.907 105.918) (end 106.907 102.496701) (width 0.25) (layer "B.Cu") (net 26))
 (segment (start 111.381 98.022701) (end 111.381 96.171) (width 0.25) (layer "B.Cu") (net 26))
 (segment (start 111.381 96.171) (end 112.556 94.996) (width 0.25) (layer "B.Cu") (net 26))
 (segment (start 116.271 96.171) (end 115.096 94.996) (width 0.25) (layer "B.Cu") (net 28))
 (segment (start 107.707 105.918) (end 107.707 104.129243) (width 0.25) (layer "B.Cu") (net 28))
 (segment (start 113.030243 98.806) (end 115.487701 98.806) (width 0.25) (layer "B.Cu") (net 28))
 (segment (start 115.487701 98.806) (end 116.271 98.022701) (width 0.25) (layer "B.Cu") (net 28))
 (segment (start 116.271 98.022701) (end 116.271 96.171) (width 0.25) (layer "B.Cu") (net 28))
 (segment (start 107.707 104.129243) (end 113.030243 98.806) (width 0.25) (layer "B.Cu") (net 28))
 (segment (start 118.811 98.105) (end 118.811 96.171) (width 0.25) (layer "B.Cu") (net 30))
 (segment (start 117.602 99.314) (end 118.811 98.105) (width 0.25) (layer "B.Cu") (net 30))
 (segment (start 118.811 96.171) (end 117.636 94.996) (width 0.25) (layer "B.Cu") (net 30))
 (segment (start 108.507 103.965639) (end 113.158639 99.314) (width 0.25) (layer "B.Cu") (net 30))
 (segment (start 108.507 105.918) (end 108.507 103.965639) (width 0.25) (layer "B.Cu") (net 30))
 (segment (start 113.158639 99.314) (end 117.602 99.314) (width 0.25) (layer "B.Cu") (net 30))
 (segment (start 121.351 96.171) (end 120.176 94.996) (width 0.25) (layer "B.Cu") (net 32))
 (segment (start 109.307 105.918) (end 109.307 103.802035) (width 0.25) (layer "B.Cu") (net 32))
 (segment (start 113.287035 99.822) (end 120.142 99.822) (width 0.25) (layer "B.Cu") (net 32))
 (segment (start 121.351 98.613) (end 121.351 96.171) (width 0.25) (layer "B.Cu") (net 32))
 (segment (start 109.307 103.802035) (end 113.287035 99.822) (width 0.25) (layer "B.Cu") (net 32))
 (segment (start 120.142 99.822) (end 121.351 98.613) (width 0.25) (layer "B.Cu") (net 32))
 (segment (start 110.107 103.638431) (end 113.415431 100.33) (width 0.25) (layer "B.Cu") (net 34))
 (segment (start 113.415431 100.33) (end 122.682 100.33) (width 0.25) (layer "B.Cu") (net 34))
 (segment (start 122.682 100.33) (end 123.891 99.121) (width 0.25) (layer "B.Cu") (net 34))
 (segment (start 123.891 96.171) (end 122.716 94.996) (width 0.25) (layer "B.Cu") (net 34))
 (segment (start 110.107 105.918) (end 110.107 103.638431) (width 0.25) (layer "B.Cu") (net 34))
 (segment (start 123.891 99.121) (end 123.891 96.171) (width 0.25) (layer "B.Cu") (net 34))
 (segment (start 113.543827 100.838) (end 125.73 100.838) (width 0.25) (layer "B.Cu") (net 36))
 (segment (start 110.907 105.918) (end 110.907 103.474827) (width 0.25) (layer "B.Cu") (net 36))
 (segment (start 125.256 94.996) (end 126.431 96.171) (width 0.25) (layer "B.Cu") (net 36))
 (segment (start 126.431 100.137) (end 125.73 100.838) (width 0.25) (layer "B.Cu") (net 36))
 (segment (start 110.907 103.474827) (end 113.543827 100.838) (width 0.25) (layer "B.Cu") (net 36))
 (segment (start 126.431 96.171) (end 126.431 100.137) (width 0.25) (layer "B.Cu") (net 36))
 (segment (start 128.971 96.171) (end 127.796 94.996) (width 0.25) (layer "B.Cu") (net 38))
 (segment (start 112.507 105.918) (end 112.507 102.511223) (width 0.25) (layer "B.Cu") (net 38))
 (segment (start 113.672223 101.346) (end 127.762 101.346) (width 0.25) (layer "B.Cu") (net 38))
 (segment (start 128.971 100.137) (end 128.971 96.171) (width 0.25) (layer "B.Cu") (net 38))
 (segment (start 112.507 105.918) (end 111.707 105.918) (width 0.25) (layer "B.Cu") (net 38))
 (segment (start 127.762 101.346) (end 128.971 100.137) (width 0.25) (layer "B.Cu") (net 38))
 (segment (start 112.507 102.511223) (end 113.672223 101.346) (width 0.25) (layer "B.Cu") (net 38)))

